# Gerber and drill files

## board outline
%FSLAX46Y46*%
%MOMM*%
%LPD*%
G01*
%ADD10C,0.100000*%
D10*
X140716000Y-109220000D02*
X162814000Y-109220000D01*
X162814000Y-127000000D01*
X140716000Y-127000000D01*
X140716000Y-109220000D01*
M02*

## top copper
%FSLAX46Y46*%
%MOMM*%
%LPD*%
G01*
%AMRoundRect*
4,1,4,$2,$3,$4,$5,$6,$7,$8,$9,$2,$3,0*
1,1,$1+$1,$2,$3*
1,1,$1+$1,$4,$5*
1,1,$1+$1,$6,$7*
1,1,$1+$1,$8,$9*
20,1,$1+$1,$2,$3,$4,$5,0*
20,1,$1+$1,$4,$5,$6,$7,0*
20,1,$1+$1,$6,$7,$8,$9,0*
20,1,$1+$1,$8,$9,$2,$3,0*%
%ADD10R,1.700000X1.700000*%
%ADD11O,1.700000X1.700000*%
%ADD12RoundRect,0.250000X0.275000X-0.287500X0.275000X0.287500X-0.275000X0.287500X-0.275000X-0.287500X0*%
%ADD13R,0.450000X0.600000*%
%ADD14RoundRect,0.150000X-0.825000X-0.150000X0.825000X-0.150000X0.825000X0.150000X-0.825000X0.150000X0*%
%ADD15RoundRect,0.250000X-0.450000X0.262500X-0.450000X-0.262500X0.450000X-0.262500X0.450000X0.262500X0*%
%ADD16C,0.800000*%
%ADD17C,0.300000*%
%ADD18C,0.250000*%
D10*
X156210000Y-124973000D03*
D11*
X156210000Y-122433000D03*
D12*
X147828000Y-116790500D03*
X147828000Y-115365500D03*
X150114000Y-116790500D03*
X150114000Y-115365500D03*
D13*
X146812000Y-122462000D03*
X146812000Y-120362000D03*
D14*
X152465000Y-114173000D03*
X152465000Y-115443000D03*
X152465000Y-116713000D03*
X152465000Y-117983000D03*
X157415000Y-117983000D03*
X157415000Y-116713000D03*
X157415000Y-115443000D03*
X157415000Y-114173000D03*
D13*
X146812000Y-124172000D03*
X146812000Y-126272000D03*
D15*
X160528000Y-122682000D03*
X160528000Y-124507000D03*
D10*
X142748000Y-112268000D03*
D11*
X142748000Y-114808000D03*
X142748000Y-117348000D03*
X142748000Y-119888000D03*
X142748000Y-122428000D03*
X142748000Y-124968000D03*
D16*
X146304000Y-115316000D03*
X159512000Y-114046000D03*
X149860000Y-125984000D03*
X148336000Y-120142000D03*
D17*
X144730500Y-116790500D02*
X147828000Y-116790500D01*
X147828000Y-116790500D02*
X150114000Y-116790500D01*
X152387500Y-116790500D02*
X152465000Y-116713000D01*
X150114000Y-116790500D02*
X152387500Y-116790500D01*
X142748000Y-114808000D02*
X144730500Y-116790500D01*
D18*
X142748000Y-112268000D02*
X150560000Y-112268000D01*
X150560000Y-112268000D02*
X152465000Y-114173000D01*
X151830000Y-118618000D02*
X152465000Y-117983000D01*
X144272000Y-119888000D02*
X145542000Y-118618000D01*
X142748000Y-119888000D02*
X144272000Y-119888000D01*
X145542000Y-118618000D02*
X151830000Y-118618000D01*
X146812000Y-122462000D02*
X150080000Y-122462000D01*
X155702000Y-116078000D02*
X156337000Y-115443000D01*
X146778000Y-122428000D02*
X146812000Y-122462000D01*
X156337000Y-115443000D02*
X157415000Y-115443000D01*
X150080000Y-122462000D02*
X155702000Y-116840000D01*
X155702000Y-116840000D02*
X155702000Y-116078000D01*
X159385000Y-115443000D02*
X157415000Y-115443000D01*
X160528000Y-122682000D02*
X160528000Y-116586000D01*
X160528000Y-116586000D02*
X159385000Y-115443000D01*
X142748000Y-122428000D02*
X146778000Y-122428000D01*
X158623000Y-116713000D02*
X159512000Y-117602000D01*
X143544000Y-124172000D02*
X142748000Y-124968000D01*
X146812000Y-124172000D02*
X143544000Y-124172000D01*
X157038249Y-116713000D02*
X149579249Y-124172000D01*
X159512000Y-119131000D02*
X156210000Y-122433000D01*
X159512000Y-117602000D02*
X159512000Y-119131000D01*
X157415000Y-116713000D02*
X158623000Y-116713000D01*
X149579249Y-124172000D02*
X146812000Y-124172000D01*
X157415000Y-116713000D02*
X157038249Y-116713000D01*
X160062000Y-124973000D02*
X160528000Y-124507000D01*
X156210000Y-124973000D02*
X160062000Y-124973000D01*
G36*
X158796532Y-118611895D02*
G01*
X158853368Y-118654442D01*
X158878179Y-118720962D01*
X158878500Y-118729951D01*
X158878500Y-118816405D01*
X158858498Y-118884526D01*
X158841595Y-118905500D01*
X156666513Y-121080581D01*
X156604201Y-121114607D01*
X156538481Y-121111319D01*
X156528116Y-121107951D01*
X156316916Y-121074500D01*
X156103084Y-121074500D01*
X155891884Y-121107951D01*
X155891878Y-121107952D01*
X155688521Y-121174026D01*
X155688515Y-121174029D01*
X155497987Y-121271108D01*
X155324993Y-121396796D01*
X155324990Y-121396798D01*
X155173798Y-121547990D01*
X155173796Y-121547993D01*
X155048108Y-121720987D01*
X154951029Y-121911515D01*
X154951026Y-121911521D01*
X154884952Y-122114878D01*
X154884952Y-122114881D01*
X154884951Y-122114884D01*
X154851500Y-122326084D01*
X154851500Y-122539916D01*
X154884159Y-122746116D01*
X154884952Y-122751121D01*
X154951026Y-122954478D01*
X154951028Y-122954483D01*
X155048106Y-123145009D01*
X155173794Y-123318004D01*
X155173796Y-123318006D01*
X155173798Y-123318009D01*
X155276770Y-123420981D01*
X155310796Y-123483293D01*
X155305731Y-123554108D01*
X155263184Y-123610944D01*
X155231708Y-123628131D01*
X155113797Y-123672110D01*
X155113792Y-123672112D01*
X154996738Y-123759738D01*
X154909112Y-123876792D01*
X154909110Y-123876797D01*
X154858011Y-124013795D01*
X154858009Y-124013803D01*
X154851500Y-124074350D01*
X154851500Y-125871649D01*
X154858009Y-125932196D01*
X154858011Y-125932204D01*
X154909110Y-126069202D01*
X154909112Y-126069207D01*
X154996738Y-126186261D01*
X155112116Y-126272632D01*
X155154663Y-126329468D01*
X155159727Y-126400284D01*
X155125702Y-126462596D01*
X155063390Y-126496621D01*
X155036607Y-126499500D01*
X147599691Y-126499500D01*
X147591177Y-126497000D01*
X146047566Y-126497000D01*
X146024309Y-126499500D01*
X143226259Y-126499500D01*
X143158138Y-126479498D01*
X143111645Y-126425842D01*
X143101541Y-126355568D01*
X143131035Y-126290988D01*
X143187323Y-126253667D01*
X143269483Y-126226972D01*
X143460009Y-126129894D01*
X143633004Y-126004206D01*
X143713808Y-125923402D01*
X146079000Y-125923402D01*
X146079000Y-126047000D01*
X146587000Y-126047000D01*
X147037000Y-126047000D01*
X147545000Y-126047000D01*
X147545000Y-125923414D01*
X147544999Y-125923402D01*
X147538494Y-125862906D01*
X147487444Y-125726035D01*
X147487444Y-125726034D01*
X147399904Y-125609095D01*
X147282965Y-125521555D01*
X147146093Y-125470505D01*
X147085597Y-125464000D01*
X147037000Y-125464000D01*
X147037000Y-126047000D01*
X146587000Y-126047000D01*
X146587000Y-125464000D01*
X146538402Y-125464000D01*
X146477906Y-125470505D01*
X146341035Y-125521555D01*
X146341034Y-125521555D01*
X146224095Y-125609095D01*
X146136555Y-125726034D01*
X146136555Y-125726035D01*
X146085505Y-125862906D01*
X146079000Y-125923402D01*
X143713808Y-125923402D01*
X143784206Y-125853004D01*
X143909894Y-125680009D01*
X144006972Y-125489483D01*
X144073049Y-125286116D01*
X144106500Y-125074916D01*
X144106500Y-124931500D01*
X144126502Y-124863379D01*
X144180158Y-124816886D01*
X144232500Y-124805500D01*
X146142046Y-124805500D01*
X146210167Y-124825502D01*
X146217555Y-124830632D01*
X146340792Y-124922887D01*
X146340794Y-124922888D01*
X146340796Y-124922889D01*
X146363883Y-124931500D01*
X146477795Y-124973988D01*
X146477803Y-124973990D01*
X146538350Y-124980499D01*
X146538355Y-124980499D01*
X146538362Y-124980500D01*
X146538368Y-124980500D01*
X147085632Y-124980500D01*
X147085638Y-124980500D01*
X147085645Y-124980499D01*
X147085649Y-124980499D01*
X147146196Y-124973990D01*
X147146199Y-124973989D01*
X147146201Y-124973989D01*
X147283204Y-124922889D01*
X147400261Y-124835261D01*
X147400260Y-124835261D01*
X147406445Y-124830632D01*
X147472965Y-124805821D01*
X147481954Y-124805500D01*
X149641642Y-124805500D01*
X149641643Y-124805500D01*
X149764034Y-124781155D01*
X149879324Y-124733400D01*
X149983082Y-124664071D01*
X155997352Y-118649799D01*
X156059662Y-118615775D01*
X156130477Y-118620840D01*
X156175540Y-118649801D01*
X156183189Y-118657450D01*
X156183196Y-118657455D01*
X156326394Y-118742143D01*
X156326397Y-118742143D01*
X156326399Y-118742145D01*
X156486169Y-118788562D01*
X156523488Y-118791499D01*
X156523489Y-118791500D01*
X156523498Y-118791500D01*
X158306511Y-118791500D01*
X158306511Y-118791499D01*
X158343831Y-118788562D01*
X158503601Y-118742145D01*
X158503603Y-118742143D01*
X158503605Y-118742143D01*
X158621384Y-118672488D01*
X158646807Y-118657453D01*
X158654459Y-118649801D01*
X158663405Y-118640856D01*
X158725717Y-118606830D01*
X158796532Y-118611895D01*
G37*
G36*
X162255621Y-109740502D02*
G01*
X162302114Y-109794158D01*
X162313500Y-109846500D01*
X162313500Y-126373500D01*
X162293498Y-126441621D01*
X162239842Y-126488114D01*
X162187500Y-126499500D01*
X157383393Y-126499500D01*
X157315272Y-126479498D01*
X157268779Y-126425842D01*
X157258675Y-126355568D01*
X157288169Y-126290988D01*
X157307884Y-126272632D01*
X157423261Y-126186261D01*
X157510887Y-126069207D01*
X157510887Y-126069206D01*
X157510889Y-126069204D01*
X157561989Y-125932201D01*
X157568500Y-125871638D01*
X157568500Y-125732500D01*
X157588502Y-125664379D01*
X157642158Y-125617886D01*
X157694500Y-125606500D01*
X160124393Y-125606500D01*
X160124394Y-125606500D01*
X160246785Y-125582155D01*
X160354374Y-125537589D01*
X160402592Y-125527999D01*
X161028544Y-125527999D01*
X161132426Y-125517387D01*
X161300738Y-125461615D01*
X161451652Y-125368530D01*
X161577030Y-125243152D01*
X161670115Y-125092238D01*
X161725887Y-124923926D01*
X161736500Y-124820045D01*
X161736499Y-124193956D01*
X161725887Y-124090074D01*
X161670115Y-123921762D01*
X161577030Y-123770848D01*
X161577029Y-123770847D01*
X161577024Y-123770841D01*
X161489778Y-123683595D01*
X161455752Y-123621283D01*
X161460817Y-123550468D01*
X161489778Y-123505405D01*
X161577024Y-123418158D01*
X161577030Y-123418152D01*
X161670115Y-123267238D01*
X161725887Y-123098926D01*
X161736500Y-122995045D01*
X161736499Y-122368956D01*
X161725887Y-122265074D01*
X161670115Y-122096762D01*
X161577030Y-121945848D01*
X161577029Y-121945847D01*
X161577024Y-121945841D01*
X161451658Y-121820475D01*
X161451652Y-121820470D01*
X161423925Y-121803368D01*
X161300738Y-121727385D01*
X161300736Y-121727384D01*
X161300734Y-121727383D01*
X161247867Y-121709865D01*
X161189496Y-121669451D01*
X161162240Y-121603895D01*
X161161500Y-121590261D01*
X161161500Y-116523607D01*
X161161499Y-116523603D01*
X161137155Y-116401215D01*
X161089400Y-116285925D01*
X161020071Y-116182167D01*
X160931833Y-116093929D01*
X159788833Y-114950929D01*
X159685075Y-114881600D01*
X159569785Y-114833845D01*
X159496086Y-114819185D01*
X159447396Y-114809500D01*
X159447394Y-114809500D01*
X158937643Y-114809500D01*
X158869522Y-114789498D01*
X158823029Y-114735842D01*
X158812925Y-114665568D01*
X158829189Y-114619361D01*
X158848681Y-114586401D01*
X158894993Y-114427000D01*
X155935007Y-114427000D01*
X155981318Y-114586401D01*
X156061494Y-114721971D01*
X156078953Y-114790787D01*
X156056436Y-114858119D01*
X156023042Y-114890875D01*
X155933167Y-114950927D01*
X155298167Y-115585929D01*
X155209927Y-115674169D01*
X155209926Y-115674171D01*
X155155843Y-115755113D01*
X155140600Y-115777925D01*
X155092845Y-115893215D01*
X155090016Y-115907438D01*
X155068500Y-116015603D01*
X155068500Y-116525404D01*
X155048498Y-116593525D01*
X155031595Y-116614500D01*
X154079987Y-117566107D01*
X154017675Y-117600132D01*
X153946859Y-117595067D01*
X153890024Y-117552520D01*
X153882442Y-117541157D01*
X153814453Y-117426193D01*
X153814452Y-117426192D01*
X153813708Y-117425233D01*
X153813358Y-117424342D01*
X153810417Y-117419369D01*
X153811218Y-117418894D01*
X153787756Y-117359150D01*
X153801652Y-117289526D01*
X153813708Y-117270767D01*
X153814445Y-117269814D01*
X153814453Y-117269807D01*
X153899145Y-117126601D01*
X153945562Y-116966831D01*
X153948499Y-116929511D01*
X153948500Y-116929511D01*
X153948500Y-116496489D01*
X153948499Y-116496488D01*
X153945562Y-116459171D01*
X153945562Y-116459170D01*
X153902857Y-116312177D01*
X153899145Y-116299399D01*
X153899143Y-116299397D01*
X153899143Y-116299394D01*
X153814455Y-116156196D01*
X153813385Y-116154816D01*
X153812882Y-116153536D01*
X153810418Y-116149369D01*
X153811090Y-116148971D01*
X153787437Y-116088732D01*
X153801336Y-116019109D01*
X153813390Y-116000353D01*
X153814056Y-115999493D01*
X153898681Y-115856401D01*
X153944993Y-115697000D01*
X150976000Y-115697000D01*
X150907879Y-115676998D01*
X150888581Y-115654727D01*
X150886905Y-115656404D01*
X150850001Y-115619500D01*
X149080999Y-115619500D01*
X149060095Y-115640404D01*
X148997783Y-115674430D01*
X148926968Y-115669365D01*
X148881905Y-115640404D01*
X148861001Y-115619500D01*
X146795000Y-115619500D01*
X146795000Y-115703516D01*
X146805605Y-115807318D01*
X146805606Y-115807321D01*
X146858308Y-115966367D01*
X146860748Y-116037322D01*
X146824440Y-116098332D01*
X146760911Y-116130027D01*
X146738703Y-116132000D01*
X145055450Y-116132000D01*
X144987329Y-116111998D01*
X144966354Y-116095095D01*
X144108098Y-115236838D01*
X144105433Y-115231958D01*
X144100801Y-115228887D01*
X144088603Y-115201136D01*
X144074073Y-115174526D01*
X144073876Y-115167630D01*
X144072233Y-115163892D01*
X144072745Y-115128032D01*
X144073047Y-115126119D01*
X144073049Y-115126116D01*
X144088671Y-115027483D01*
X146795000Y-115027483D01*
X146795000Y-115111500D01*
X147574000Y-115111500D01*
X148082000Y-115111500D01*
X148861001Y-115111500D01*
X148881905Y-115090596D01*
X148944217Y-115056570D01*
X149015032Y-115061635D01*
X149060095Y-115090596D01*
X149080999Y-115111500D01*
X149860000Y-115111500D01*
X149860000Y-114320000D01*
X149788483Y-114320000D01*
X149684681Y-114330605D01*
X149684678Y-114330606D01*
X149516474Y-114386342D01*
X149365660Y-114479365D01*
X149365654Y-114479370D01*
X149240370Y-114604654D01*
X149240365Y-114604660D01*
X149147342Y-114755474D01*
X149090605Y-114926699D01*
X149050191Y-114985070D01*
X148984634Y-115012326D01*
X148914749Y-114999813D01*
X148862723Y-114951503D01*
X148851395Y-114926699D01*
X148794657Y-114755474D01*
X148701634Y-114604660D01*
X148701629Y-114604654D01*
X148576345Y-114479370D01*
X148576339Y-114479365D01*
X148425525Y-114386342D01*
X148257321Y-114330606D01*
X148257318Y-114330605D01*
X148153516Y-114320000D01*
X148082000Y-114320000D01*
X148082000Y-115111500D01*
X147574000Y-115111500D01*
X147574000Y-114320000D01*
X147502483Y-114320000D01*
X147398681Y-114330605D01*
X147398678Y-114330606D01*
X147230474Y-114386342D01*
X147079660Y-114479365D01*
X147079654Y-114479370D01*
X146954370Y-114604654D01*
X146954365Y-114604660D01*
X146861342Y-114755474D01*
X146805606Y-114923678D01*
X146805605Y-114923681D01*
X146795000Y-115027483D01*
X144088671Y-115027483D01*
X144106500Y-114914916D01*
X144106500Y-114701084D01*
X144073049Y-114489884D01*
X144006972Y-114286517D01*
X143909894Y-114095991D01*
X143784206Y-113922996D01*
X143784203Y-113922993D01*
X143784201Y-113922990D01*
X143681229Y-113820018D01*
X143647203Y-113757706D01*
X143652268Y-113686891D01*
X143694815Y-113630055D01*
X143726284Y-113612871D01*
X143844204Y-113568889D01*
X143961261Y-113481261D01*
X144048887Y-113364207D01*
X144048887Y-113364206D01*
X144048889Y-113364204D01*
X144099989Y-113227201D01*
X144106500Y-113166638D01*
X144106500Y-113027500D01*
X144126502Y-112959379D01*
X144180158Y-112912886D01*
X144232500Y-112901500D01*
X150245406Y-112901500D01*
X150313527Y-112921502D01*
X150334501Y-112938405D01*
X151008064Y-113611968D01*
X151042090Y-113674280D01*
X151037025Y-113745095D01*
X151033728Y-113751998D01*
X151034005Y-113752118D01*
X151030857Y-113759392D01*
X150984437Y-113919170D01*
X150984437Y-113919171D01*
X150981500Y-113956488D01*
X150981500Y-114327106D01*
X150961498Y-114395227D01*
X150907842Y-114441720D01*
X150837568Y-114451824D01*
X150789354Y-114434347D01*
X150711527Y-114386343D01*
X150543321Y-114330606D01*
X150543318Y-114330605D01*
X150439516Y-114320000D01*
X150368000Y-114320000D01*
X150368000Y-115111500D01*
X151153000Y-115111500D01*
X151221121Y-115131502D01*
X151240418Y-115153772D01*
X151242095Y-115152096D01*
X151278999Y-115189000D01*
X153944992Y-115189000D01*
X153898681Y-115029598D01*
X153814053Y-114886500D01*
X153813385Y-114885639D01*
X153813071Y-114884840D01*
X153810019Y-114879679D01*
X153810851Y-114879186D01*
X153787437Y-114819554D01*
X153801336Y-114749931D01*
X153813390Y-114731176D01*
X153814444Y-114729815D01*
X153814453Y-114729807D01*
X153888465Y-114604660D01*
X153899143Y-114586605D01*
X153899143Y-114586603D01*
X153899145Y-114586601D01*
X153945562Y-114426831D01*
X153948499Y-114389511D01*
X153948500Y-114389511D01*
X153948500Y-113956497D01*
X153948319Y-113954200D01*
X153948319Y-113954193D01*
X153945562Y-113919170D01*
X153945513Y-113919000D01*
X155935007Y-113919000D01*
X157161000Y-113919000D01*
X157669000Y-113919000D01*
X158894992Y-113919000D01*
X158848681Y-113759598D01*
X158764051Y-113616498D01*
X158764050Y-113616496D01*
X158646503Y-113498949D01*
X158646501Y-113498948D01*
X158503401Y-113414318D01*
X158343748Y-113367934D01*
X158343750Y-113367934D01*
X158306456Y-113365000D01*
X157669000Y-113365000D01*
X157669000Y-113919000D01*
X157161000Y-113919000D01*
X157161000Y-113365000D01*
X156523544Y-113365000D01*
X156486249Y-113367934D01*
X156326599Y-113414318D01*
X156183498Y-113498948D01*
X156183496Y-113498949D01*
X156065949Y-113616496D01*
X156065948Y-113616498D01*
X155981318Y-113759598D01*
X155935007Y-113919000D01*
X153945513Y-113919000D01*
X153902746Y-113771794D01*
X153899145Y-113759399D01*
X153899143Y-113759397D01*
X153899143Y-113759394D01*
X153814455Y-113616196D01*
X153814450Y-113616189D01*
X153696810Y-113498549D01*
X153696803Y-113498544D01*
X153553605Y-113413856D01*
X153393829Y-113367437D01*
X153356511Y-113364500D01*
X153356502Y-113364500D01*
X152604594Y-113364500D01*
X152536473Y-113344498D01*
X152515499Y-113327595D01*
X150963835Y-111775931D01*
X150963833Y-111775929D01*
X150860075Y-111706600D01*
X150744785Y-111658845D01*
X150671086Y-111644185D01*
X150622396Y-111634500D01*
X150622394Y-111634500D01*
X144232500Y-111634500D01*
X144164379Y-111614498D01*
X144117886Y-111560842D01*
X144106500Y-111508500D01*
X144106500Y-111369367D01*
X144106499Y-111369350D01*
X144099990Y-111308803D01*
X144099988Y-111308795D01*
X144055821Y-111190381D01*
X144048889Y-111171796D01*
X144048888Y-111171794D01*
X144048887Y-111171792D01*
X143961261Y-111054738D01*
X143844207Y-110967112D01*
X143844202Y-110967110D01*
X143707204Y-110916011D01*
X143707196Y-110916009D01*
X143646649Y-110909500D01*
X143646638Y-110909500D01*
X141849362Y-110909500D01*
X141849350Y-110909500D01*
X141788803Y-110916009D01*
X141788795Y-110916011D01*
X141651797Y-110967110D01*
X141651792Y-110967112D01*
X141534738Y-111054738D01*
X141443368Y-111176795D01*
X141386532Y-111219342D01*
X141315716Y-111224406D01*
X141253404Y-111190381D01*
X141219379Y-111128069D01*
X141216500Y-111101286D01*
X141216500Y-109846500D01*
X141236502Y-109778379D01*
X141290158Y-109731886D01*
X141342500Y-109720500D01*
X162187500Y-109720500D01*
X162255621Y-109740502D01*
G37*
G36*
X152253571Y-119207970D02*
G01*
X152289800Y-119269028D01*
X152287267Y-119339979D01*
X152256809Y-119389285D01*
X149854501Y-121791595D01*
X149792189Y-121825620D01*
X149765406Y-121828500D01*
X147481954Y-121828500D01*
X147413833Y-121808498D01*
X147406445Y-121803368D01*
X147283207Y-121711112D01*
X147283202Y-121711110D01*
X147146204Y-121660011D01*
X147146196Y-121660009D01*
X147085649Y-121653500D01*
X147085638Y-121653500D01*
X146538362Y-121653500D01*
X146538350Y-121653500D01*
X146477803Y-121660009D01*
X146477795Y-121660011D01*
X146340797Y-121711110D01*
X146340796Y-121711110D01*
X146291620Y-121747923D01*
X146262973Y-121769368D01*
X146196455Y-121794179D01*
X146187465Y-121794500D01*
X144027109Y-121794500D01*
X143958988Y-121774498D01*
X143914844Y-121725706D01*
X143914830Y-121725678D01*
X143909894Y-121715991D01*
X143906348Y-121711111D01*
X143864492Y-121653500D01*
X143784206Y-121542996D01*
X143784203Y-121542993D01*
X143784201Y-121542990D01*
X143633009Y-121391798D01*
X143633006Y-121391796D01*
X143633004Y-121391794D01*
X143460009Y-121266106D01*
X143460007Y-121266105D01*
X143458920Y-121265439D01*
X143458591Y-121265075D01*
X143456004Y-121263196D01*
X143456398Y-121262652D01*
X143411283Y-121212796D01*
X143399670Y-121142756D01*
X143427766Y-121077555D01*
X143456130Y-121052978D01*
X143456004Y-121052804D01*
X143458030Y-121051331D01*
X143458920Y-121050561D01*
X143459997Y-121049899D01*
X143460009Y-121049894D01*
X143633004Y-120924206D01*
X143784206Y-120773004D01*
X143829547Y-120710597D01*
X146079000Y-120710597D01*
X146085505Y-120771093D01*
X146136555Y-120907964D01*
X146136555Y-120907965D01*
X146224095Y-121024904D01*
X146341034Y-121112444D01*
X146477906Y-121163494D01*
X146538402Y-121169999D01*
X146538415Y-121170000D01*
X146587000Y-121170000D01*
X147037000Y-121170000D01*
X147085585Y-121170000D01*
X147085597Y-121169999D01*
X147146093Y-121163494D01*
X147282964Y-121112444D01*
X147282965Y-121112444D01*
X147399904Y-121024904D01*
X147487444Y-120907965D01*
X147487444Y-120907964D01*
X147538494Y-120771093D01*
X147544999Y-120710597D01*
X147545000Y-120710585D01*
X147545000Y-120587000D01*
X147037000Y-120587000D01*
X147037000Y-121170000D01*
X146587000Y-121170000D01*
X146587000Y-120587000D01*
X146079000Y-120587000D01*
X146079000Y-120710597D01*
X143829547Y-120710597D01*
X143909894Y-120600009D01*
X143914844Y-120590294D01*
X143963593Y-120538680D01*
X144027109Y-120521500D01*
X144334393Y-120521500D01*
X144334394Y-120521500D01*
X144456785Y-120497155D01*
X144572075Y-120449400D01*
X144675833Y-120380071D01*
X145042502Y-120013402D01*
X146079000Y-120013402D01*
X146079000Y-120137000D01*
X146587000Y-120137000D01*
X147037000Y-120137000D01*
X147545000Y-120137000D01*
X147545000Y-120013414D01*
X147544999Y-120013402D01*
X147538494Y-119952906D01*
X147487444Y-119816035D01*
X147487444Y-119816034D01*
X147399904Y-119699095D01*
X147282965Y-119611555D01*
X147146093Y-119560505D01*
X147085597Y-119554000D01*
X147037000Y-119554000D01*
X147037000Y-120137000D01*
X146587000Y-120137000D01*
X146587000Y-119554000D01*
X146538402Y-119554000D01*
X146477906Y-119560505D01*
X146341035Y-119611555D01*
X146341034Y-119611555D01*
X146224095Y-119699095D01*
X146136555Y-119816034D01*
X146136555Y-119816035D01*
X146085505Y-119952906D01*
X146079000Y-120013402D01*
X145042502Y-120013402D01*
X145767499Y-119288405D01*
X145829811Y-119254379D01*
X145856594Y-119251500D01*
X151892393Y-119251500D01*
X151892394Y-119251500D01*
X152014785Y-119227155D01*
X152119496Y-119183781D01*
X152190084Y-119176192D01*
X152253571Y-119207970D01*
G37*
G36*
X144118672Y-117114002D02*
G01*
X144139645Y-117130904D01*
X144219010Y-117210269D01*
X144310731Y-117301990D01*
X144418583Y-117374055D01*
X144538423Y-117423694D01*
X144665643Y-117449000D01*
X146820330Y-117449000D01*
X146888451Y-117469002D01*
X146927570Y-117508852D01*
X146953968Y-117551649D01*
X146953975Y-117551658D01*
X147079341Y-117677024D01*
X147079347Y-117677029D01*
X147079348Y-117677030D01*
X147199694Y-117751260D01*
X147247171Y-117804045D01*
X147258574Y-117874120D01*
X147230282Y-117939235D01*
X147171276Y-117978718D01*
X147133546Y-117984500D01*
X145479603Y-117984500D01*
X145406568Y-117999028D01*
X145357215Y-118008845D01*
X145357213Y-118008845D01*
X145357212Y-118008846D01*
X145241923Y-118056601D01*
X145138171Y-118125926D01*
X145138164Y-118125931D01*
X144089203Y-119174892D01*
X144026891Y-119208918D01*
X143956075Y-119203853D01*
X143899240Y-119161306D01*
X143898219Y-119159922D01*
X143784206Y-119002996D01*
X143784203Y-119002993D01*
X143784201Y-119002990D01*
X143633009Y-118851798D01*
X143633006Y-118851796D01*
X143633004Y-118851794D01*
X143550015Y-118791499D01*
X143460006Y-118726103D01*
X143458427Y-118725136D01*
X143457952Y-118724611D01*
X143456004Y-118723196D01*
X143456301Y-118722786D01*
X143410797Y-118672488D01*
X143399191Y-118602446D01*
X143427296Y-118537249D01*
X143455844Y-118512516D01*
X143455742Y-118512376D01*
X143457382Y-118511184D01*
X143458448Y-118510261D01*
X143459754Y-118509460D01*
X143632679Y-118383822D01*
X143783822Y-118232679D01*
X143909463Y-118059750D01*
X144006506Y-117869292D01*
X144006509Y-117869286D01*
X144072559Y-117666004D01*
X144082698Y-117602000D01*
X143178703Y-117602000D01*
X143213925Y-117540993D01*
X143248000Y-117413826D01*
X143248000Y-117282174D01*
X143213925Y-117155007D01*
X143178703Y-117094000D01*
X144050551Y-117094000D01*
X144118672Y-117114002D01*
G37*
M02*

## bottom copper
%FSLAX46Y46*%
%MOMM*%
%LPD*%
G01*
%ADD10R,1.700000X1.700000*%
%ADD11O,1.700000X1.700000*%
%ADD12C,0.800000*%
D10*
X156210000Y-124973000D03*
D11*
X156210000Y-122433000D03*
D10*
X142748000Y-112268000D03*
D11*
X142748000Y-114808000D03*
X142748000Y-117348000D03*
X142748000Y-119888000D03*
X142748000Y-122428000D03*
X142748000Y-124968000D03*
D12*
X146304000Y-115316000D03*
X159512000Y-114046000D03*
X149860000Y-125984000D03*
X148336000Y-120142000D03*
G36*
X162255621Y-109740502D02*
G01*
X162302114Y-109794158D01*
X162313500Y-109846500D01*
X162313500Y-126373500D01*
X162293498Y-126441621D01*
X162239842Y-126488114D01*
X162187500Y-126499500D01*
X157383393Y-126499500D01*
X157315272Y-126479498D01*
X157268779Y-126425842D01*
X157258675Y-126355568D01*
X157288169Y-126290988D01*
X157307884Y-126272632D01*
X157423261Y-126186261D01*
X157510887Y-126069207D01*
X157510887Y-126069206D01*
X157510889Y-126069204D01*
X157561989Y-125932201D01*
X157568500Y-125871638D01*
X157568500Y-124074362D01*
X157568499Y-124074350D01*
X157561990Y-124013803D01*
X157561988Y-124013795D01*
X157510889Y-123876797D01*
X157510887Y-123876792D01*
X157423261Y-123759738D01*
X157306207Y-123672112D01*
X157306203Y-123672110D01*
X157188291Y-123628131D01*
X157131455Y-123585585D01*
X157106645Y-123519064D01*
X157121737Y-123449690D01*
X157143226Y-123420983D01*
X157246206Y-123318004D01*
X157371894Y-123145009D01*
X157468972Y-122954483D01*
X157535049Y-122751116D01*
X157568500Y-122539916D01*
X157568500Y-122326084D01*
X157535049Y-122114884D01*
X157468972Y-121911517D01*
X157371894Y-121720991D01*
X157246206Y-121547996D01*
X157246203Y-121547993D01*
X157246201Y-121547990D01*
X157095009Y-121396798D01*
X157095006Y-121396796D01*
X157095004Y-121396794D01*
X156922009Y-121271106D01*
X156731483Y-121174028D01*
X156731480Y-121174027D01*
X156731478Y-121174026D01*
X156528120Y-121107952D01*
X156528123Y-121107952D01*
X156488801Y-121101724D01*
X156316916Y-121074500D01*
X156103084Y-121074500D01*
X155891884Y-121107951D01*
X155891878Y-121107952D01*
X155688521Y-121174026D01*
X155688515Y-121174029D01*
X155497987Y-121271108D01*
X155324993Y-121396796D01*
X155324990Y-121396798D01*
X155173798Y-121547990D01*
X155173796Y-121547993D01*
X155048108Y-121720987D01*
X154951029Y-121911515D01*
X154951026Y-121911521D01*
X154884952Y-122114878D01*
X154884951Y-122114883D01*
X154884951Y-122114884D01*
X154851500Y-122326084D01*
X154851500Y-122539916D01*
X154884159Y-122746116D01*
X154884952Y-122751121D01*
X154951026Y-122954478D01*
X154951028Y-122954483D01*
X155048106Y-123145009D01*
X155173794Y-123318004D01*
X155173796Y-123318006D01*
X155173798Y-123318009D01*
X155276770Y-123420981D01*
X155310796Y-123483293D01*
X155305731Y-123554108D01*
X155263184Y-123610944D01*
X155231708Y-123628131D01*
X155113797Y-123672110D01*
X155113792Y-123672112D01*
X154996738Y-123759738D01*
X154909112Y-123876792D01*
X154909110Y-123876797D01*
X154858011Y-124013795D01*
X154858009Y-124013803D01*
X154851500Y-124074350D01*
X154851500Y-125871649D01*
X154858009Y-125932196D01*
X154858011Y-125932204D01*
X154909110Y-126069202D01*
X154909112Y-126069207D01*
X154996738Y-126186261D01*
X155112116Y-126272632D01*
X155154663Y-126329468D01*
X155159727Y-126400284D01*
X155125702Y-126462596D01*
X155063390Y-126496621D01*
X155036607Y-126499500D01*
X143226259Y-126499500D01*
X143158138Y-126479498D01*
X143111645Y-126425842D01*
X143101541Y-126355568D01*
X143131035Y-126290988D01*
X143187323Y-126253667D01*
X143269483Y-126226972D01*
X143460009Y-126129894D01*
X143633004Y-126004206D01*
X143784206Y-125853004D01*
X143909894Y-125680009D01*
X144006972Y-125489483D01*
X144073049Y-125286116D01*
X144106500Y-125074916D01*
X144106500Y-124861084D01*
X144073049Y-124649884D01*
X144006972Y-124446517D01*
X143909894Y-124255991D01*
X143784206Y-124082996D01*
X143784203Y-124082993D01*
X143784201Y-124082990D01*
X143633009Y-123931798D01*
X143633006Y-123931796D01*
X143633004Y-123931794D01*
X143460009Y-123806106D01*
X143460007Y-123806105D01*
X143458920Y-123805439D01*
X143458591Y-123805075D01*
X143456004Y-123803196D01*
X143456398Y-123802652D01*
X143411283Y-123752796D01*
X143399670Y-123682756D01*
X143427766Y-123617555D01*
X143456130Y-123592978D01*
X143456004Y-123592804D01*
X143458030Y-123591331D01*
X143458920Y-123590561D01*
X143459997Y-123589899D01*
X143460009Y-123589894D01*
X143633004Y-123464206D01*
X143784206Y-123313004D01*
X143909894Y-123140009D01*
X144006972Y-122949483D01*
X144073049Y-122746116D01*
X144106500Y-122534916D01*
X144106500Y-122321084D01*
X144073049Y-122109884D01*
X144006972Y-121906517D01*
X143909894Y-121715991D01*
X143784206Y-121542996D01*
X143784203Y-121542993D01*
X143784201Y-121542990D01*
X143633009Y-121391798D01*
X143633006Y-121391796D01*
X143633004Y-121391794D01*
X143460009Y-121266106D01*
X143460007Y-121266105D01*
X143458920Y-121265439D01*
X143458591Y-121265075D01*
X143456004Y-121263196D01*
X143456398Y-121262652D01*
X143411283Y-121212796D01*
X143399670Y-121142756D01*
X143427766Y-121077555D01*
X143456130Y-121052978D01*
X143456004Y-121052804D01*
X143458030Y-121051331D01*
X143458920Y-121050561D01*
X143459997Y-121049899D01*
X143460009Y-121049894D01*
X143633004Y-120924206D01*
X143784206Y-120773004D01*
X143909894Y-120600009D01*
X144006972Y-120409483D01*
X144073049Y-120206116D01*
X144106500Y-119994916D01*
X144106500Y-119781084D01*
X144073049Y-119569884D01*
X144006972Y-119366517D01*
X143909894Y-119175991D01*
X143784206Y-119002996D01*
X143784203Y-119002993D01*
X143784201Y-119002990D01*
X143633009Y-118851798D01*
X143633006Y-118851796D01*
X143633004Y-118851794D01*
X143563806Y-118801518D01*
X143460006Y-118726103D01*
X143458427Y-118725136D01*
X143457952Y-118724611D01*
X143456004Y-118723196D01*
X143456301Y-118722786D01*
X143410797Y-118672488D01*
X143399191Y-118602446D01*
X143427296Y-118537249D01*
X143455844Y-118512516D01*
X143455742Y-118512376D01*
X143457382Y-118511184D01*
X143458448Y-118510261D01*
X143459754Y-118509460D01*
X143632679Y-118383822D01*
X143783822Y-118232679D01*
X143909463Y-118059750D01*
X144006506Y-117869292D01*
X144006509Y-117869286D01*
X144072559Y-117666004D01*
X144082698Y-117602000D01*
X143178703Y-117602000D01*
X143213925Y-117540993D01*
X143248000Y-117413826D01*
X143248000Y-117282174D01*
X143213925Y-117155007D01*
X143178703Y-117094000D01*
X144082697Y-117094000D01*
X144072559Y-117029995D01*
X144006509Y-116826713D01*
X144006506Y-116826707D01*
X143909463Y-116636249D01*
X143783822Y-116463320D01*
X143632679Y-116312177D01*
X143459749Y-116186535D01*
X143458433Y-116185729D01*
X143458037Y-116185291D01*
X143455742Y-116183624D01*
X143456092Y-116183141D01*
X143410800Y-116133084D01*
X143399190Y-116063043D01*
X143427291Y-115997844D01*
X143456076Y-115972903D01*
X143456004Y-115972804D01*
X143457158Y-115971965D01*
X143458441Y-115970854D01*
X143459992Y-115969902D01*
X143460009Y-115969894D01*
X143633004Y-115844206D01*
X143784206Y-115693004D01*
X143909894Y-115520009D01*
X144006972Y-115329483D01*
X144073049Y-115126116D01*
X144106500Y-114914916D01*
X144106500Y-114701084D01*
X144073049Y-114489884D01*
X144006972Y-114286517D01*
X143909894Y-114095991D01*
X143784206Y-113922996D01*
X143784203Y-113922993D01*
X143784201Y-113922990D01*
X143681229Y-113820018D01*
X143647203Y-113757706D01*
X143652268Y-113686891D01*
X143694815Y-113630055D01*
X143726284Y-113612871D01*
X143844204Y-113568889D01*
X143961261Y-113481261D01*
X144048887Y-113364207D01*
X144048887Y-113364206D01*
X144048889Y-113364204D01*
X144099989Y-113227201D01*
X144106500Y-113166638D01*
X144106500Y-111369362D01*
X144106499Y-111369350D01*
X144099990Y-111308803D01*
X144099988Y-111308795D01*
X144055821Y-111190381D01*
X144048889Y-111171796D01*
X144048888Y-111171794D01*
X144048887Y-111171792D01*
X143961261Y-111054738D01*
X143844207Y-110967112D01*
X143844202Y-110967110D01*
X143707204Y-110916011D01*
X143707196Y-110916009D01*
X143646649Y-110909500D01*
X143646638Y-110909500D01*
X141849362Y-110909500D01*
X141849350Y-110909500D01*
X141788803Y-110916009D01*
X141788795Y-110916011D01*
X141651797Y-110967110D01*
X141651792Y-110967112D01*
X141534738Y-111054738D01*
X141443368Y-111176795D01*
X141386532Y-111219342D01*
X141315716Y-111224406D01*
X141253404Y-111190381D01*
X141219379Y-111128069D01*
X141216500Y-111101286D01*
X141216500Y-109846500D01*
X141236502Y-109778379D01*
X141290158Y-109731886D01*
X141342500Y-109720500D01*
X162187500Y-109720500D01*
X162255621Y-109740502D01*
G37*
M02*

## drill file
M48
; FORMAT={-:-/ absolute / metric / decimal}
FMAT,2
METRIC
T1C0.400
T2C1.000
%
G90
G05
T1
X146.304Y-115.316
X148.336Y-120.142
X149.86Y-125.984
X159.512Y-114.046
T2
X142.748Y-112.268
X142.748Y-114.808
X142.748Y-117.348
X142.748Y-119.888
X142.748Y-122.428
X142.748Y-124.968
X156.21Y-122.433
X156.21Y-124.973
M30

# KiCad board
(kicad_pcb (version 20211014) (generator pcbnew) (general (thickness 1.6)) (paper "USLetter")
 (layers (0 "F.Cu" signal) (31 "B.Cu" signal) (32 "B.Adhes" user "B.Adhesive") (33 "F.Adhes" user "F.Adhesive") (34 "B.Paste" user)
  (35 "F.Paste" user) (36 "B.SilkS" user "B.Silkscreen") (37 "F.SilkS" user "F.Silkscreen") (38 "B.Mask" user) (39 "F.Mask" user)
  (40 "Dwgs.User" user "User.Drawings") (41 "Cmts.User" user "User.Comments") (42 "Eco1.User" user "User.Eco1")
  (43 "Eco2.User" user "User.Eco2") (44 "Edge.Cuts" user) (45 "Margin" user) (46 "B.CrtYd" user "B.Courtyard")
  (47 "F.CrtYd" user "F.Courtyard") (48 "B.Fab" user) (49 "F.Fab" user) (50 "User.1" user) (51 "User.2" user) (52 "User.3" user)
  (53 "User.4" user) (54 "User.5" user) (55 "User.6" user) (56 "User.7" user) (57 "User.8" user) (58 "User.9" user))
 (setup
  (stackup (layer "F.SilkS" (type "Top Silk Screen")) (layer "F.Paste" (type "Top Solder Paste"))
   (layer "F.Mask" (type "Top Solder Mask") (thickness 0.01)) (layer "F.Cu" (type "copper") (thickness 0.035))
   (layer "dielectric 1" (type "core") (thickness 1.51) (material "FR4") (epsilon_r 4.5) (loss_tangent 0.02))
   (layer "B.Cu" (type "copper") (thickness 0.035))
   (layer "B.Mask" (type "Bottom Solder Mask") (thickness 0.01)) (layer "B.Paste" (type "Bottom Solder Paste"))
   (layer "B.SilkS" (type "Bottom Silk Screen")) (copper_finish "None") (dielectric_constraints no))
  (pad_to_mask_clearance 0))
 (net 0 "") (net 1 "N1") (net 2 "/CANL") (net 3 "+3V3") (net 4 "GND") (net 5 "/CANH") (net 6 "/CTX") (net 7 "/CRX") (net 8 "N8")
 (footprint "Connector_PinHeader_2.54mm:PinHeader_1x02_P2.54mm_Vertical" (layer "F.Cu") (at 156.21 124.973 180)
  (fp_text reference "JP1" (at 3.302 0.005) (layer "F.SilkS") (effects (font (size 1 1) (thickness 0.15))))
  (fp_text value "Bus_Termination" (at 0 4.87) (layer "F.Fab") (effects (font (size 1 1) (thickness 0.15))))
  (pad "1" thru_hole rect (at 0 0 180) (size 1.7 1.7) (drill 1) (layers *.Cu *.Mask) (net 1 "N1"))
  (pad "2" thru_hole oval (at 0 2.54 180) (size 1.7 1.7) (drill 1) (layers *.Cu *.Mask) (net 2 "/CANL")))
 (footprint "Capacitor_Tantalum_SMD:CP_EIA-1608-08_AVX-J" (layer "F.Cu") (at 147.828 116.078 90)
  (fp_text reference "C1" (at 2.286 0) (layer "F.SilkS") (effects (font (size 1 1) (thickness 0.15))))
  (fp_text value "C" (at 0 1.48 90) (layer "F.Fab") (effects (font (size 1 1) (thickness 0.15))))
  (pad "1" smd roundrect (at -0.7125 0 90) (size 1.075 1.05) (layers "F.Cu" "F.Paste" "F.Mask") (roundrect_rratio 0.238095) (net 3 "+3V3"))
  (pad "2" smd roundrect (at 0.7125 0 90) (size 1.075 1.05) (layers "F.Cu" "F.Paste" "F.Mask") (roundrect_rratio 0.238095) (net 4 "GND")))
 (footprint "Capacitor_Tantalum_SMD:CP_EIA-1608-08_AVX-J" (layer "F.Cu") (at 150.114 116.078 90)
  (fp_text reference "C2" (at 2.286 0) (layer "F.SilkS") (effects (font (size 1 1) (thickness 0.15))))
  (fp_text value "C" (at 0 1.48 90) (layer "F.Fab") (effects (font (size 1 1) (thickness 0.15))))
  (pad "1" smd roundrect (at -0.7125 0 90) (size 1.075 1.05) (layers "F.Cu" "F.Paste" "F.Mask") (roundrect_rratio 0.238095) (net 3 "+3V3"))
  (pad "2" smd roundrect (at 0.7125 0 90) (size 1.075 1.05) (layers "F.Cu" "F.Paste" "F.Mask") (roundrect_rratio 0.238095) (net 4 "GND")))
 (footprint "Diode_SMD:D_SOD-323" (layer "F.Cu") (at 146.812 121.412 90)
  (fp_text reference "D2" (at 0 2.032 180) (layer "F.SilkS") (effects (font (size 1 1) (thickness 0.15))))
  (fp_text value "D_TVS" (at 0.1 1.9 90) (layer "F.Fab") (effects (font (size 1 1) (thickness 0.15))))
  (pad "1" smd rect (at -1.05 0 90) (size 0.6 0.45) (layers "F.Cu" "F.Paste" "F.Mask") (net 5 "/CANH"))
  (pad "2" smd rect (at 1.05 0 90) (size 0.6 0.45) (layers "F.Cu" "F.Paste" "F.Mask") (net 4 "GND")))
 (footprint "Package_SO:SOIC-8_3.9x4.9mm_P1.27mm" (layer "F.Cu") (at 154.94 116.078)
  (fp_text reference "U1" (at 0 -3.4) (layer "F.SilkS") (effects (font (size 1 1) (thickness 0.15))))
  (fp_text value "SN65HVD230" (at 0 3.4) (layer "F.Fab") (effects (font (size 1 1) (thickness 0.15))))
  (pad "1" smd roundrect (at -2.475 -1.905) (size 1.95 0.6) (layers "F.Cu" "F.Paste" "F.Mask") (roundrect_rratio 0.25) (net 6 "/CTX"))
  (pad "2" smd roundrect (at -2.475 -0.635) (size 1.95 0.6) (layers "F.Cu" "F.Paste" "F.Mask") (roundrect_rratio 0.25) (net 4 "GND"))
  (pad "3" smd roundrect (at -2.475 0.635) (size 1.95 0.6) (layers "F.Cu" "F.Paste" "F.Mask") (roundrect_rratio 0.25) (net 3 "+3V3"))
  (pad "4" smd roundrect (at -2.475 1.905) (size 1.95 0.6) (layers "F.Cu" "F.Paste" "F.Mask") (roundrect_rratio 0.25) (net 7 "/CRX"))
  (pad "5" smd roundrect (at 2.475 1.905) (size 1.95 0.6) (layers "F.Cu" "F.Paste" "F.Mask") (roundrect_rratio 0.25) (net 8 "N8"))
  (pad "6" smd roundrect (at 2.475 0.635) (size 1.95 0.6) (layers "F.Cu" "F.Paste" "F.Mask") (roundrect_rratio 0.25) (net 2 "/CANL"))
  (pad "7" smd roundrect (at 2.475 -0.635) (size 1.95 0.6) (layers "F.Cu" "F.Paste" "F.Mask") (roundrect_rratio 0.25) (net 5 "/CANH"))
  (pad "8" smd roundrect (at 2.475 -1.905) (size 1.95 0.6) (layers "F.Cu" "F.Paste" "F.Mask") (roundrect_rratio 0.25) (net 4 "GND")))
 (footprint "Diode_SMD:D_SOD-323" (layer "F.Cu") (at 146.812 125.222 -90)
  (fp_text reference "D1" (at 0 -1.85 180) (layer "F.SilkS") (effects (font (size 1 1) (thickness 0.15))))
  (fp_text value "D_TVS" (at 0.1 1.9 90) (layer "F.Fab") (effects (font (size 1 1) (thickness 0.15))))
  (pad "1" smd rect (at -1.05 0 270) (size 0.6 0.45) (layers "F.Cu" "F.Paste" "F.Mask") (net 2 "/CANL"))
  (pad "2" smd rect (at 1.05 0 270) (size 0.6 0.45) (layers "F.Cu" "F.Paste" "F.Mask") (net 4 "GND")))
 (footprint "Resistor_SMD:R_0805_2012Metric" (layer "F.Cu") (at 160.528 123.5945 -90)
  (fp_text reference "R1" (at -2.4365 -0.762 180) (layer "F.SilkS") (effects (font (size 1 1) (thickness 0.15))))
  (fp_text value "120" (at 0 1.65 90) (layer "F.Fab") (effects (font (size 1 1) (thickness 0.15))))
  (pad "1" smd roundrect (at -0.9125 0 270) (size 1.025 1.4) (layers "F.Cu" "F.Paste" "F.Mask") (roundrect_rratio 0.243902) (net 5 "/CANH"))
  (pad "2" smd roundrect (at 0.9125 0 270) (size 1.025 1.4) (layers "F.Cu" "F.Paste" "F.Mask") (roundrect_rratio 0.243902) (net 1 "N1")))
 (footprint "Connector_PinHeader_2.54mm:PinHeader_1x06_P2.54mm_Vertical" (layer "B.Cu") (at 142.748 112.268 180)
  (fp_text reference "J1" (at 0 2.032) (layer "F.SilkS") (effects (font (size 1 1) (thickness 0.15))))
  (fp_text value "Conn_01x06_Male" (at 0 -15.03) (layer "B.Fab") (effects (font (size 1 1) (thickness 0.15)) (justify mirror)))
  (pad "1" thru_hole rect (at 0 0 180) (size 1.7 1.7) (drill 1) (layers *.Cu *.Mask) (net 6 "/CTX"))
  (pad "2" thru_hole oval (at 0 -2.54 180) (size 1.7 1.7) (drill 1) (layers *.Cu *.Mask) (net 3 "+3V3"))
  (pad "3" thru_hole oval (at 0 -5.08 180) (size 1.7 1.7) (drill 1) (layers *.Cu *.Mask) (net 4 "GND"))
  (pad "4" thru_hole oval (at 0 -7.62 180) (size 1.7 1.7) (drill 1) (layers *.Cu *.Mask) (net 7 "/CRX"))
  (pad "5" thru_hole oval (at 0 -10.16 180) (size 1.7 1.7) (drill 1) (layers *.Cu *.Mask) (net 5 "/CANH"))
  (pad "6" thru_hole oval (at 0 -12.7 180) (size 1.7 1.7) (drill 1) (layers *.Cu *.Mask) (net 2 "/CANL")))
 (gr_rect (start 140.716 127) (end 162.814 109.22) (layer "Edge.Cuts") (width 0.1) (fill none))
 (segment (start 144.7305 116.7905) (end 147.828 116.7905) (width 0.3) (layer "F.Cu") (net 3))
 (segment (start 147.828 116.7905) (end 150.114 116.7905) (width 0.3) (layer "F.Cu") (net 3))
 (segment (start 152.3875 116.7905) (end 152.465 116.713) (width 0.3) (layer "F.Cu") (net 3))
 (segment (start 150.114 116.7905) (end 152.3875 116.7905) (width 0.3) (layer "F.Cu") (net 3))
 (segment (start 142.748 114.808) (end 144.7305 116.7905) (width 0.3) (layer "F.Cu") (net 3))
 (via (at 146.304 115.316) (size 0.8) (drill 0.4) (layers "F.Cu" "B.Cu") (free) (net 4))
 (via (at 159.512 114.046) (size 0.8) (drill 0.4) (layers "F.Cu" "B.Cu") (free) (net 4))
 (via (at 149.86 125.984) (size 0.8) (drill 0.4) (layers "F.Cu" "B.Cu") (free) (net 4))
 (via (at 148.336 120.142) (size 0.8) (drill 0.4) (layers "F.Cu" "B.Cu") (free) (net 4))
 (segment (start 142.748 112.268) (end 150.56 112.268) (width 0.25) (layer "F.Cu") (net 6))
 (segment (start 150.56 112.268) (end 152.465 114.173) (width 0.25) (layer "F.Cu") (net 6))
 (segment (start 151.83 118.618) (end 152.465 117.983) (width 0.25) (layer "F.Cu") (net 7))
 (segment (start 144.272 119.888) (end 145.542 118.618) (width 0.25) (layer "F.Cu") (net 7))
 (segment (start 142.748 119.888) (end 144.272 119.888) (width 0.25) (layer "F.Cu") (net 7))
 (segment (start 145.542 118.618) (end 151.83 118.618) (width 0.25) (layer "F.Cu") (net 7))
 (segment (start 146.812 122.462) (end 150.08 122.462) (width 0.25) (layer "F.Cu") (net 5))
 (segment (start 155.702 116.078) (end 156.337 115.443) (width 0.25) (layer "F.Cu") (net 5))
 (segment (start 146.778 122.428) (end 146.812 122.462) (width 0.25) (layer "F.Cu") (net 5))
 (segment (start 156.337 115.443) (end 157.415 115.443) (width 0.25) (layer "F.Cu") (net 5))
 (segment (start 150.08 122.462) (end 155.702 116.84) (width 0.25) (layer "F.Cu") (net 5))
 (segment (start 155.702 116.84) (end 155.702 116.078) (width 0.25) (layer "F.Cu") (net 5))
 (segment (start 159.385 115.443) (end 157.415 115.443) (width 0.25) (layer "F.Cu") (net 5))
 (segment (start 160.528 122.682) (end 160.528 116.586) (width 0.25) (layer "F.Cu") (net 5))
 (segment (start 160.528 116.586) (end 159.385 115.443) (width 0.25) (layer "F.Cu") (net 5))
 (segment (start 142.748 122.428) (end 146.778 122.428) (width 0.25) (layer "F.Cu") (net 5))
 (segment (start 158.623 116.713) (end 159.512 117.602) (width 0.25) (layer "F.Cu") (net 2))
 (segment (start 143.544 124.172) (end 142.748 124.968) (width 0.25) (layer "F.Cu") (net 2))
 (segment (start 146.812 124.172) (end 143.544 124.172) (width 0.25) (layer "F.Cu") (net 2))
 (segment (start 157.038249 116.713) (end 149.579249 124.172) (width 0.25) (layer "F.Cu") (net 2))
 (segment (start 159.512 119.131) (end 156.21 122.433) (width 0.25) (layer "F.Cu") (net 2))
 (segment (start 159.512 117.602) (end 159.512 119.131) (width 0.25) (layer "F.Cu") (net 2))
 (segment (start 157.415 116.713) (end 158.623 116.713) (width 0.25) (layer "F.Cu") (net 2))
 (segment (start 149.579249 124.172) (end 146.812 124.172) (width 0.25) (layer "F.Cu") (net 2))
 (segment (start 157.415 116.713) (end 157.038249 116.713) (width 0.25) (layer "F.Cu") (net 2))
 (segment (start 160.062 124.973) (end 160.528 124.507) (width 0.25) (layer "F.Cu") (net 1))
 (segment (start 156.21 124.973) (end 160.062 124.973) (width 0.25) (layer "F.Cu") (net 1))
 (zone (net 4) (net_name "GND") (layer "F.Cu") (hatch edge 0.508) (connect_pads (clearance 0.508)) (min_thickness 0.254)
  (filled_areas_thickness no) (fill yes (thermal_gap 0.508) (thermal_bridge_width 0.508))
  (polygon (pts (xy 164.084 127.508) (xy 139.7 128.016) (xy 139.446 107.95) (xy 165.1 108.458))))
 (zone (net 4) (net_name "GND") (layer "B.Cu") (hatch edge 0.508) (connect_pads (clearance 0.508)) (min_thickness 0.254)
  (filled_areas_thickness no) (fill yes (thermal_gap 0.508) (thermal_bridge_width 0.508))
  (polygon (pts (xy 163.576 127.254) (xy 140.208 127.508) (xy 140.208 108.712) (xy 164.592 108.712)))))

